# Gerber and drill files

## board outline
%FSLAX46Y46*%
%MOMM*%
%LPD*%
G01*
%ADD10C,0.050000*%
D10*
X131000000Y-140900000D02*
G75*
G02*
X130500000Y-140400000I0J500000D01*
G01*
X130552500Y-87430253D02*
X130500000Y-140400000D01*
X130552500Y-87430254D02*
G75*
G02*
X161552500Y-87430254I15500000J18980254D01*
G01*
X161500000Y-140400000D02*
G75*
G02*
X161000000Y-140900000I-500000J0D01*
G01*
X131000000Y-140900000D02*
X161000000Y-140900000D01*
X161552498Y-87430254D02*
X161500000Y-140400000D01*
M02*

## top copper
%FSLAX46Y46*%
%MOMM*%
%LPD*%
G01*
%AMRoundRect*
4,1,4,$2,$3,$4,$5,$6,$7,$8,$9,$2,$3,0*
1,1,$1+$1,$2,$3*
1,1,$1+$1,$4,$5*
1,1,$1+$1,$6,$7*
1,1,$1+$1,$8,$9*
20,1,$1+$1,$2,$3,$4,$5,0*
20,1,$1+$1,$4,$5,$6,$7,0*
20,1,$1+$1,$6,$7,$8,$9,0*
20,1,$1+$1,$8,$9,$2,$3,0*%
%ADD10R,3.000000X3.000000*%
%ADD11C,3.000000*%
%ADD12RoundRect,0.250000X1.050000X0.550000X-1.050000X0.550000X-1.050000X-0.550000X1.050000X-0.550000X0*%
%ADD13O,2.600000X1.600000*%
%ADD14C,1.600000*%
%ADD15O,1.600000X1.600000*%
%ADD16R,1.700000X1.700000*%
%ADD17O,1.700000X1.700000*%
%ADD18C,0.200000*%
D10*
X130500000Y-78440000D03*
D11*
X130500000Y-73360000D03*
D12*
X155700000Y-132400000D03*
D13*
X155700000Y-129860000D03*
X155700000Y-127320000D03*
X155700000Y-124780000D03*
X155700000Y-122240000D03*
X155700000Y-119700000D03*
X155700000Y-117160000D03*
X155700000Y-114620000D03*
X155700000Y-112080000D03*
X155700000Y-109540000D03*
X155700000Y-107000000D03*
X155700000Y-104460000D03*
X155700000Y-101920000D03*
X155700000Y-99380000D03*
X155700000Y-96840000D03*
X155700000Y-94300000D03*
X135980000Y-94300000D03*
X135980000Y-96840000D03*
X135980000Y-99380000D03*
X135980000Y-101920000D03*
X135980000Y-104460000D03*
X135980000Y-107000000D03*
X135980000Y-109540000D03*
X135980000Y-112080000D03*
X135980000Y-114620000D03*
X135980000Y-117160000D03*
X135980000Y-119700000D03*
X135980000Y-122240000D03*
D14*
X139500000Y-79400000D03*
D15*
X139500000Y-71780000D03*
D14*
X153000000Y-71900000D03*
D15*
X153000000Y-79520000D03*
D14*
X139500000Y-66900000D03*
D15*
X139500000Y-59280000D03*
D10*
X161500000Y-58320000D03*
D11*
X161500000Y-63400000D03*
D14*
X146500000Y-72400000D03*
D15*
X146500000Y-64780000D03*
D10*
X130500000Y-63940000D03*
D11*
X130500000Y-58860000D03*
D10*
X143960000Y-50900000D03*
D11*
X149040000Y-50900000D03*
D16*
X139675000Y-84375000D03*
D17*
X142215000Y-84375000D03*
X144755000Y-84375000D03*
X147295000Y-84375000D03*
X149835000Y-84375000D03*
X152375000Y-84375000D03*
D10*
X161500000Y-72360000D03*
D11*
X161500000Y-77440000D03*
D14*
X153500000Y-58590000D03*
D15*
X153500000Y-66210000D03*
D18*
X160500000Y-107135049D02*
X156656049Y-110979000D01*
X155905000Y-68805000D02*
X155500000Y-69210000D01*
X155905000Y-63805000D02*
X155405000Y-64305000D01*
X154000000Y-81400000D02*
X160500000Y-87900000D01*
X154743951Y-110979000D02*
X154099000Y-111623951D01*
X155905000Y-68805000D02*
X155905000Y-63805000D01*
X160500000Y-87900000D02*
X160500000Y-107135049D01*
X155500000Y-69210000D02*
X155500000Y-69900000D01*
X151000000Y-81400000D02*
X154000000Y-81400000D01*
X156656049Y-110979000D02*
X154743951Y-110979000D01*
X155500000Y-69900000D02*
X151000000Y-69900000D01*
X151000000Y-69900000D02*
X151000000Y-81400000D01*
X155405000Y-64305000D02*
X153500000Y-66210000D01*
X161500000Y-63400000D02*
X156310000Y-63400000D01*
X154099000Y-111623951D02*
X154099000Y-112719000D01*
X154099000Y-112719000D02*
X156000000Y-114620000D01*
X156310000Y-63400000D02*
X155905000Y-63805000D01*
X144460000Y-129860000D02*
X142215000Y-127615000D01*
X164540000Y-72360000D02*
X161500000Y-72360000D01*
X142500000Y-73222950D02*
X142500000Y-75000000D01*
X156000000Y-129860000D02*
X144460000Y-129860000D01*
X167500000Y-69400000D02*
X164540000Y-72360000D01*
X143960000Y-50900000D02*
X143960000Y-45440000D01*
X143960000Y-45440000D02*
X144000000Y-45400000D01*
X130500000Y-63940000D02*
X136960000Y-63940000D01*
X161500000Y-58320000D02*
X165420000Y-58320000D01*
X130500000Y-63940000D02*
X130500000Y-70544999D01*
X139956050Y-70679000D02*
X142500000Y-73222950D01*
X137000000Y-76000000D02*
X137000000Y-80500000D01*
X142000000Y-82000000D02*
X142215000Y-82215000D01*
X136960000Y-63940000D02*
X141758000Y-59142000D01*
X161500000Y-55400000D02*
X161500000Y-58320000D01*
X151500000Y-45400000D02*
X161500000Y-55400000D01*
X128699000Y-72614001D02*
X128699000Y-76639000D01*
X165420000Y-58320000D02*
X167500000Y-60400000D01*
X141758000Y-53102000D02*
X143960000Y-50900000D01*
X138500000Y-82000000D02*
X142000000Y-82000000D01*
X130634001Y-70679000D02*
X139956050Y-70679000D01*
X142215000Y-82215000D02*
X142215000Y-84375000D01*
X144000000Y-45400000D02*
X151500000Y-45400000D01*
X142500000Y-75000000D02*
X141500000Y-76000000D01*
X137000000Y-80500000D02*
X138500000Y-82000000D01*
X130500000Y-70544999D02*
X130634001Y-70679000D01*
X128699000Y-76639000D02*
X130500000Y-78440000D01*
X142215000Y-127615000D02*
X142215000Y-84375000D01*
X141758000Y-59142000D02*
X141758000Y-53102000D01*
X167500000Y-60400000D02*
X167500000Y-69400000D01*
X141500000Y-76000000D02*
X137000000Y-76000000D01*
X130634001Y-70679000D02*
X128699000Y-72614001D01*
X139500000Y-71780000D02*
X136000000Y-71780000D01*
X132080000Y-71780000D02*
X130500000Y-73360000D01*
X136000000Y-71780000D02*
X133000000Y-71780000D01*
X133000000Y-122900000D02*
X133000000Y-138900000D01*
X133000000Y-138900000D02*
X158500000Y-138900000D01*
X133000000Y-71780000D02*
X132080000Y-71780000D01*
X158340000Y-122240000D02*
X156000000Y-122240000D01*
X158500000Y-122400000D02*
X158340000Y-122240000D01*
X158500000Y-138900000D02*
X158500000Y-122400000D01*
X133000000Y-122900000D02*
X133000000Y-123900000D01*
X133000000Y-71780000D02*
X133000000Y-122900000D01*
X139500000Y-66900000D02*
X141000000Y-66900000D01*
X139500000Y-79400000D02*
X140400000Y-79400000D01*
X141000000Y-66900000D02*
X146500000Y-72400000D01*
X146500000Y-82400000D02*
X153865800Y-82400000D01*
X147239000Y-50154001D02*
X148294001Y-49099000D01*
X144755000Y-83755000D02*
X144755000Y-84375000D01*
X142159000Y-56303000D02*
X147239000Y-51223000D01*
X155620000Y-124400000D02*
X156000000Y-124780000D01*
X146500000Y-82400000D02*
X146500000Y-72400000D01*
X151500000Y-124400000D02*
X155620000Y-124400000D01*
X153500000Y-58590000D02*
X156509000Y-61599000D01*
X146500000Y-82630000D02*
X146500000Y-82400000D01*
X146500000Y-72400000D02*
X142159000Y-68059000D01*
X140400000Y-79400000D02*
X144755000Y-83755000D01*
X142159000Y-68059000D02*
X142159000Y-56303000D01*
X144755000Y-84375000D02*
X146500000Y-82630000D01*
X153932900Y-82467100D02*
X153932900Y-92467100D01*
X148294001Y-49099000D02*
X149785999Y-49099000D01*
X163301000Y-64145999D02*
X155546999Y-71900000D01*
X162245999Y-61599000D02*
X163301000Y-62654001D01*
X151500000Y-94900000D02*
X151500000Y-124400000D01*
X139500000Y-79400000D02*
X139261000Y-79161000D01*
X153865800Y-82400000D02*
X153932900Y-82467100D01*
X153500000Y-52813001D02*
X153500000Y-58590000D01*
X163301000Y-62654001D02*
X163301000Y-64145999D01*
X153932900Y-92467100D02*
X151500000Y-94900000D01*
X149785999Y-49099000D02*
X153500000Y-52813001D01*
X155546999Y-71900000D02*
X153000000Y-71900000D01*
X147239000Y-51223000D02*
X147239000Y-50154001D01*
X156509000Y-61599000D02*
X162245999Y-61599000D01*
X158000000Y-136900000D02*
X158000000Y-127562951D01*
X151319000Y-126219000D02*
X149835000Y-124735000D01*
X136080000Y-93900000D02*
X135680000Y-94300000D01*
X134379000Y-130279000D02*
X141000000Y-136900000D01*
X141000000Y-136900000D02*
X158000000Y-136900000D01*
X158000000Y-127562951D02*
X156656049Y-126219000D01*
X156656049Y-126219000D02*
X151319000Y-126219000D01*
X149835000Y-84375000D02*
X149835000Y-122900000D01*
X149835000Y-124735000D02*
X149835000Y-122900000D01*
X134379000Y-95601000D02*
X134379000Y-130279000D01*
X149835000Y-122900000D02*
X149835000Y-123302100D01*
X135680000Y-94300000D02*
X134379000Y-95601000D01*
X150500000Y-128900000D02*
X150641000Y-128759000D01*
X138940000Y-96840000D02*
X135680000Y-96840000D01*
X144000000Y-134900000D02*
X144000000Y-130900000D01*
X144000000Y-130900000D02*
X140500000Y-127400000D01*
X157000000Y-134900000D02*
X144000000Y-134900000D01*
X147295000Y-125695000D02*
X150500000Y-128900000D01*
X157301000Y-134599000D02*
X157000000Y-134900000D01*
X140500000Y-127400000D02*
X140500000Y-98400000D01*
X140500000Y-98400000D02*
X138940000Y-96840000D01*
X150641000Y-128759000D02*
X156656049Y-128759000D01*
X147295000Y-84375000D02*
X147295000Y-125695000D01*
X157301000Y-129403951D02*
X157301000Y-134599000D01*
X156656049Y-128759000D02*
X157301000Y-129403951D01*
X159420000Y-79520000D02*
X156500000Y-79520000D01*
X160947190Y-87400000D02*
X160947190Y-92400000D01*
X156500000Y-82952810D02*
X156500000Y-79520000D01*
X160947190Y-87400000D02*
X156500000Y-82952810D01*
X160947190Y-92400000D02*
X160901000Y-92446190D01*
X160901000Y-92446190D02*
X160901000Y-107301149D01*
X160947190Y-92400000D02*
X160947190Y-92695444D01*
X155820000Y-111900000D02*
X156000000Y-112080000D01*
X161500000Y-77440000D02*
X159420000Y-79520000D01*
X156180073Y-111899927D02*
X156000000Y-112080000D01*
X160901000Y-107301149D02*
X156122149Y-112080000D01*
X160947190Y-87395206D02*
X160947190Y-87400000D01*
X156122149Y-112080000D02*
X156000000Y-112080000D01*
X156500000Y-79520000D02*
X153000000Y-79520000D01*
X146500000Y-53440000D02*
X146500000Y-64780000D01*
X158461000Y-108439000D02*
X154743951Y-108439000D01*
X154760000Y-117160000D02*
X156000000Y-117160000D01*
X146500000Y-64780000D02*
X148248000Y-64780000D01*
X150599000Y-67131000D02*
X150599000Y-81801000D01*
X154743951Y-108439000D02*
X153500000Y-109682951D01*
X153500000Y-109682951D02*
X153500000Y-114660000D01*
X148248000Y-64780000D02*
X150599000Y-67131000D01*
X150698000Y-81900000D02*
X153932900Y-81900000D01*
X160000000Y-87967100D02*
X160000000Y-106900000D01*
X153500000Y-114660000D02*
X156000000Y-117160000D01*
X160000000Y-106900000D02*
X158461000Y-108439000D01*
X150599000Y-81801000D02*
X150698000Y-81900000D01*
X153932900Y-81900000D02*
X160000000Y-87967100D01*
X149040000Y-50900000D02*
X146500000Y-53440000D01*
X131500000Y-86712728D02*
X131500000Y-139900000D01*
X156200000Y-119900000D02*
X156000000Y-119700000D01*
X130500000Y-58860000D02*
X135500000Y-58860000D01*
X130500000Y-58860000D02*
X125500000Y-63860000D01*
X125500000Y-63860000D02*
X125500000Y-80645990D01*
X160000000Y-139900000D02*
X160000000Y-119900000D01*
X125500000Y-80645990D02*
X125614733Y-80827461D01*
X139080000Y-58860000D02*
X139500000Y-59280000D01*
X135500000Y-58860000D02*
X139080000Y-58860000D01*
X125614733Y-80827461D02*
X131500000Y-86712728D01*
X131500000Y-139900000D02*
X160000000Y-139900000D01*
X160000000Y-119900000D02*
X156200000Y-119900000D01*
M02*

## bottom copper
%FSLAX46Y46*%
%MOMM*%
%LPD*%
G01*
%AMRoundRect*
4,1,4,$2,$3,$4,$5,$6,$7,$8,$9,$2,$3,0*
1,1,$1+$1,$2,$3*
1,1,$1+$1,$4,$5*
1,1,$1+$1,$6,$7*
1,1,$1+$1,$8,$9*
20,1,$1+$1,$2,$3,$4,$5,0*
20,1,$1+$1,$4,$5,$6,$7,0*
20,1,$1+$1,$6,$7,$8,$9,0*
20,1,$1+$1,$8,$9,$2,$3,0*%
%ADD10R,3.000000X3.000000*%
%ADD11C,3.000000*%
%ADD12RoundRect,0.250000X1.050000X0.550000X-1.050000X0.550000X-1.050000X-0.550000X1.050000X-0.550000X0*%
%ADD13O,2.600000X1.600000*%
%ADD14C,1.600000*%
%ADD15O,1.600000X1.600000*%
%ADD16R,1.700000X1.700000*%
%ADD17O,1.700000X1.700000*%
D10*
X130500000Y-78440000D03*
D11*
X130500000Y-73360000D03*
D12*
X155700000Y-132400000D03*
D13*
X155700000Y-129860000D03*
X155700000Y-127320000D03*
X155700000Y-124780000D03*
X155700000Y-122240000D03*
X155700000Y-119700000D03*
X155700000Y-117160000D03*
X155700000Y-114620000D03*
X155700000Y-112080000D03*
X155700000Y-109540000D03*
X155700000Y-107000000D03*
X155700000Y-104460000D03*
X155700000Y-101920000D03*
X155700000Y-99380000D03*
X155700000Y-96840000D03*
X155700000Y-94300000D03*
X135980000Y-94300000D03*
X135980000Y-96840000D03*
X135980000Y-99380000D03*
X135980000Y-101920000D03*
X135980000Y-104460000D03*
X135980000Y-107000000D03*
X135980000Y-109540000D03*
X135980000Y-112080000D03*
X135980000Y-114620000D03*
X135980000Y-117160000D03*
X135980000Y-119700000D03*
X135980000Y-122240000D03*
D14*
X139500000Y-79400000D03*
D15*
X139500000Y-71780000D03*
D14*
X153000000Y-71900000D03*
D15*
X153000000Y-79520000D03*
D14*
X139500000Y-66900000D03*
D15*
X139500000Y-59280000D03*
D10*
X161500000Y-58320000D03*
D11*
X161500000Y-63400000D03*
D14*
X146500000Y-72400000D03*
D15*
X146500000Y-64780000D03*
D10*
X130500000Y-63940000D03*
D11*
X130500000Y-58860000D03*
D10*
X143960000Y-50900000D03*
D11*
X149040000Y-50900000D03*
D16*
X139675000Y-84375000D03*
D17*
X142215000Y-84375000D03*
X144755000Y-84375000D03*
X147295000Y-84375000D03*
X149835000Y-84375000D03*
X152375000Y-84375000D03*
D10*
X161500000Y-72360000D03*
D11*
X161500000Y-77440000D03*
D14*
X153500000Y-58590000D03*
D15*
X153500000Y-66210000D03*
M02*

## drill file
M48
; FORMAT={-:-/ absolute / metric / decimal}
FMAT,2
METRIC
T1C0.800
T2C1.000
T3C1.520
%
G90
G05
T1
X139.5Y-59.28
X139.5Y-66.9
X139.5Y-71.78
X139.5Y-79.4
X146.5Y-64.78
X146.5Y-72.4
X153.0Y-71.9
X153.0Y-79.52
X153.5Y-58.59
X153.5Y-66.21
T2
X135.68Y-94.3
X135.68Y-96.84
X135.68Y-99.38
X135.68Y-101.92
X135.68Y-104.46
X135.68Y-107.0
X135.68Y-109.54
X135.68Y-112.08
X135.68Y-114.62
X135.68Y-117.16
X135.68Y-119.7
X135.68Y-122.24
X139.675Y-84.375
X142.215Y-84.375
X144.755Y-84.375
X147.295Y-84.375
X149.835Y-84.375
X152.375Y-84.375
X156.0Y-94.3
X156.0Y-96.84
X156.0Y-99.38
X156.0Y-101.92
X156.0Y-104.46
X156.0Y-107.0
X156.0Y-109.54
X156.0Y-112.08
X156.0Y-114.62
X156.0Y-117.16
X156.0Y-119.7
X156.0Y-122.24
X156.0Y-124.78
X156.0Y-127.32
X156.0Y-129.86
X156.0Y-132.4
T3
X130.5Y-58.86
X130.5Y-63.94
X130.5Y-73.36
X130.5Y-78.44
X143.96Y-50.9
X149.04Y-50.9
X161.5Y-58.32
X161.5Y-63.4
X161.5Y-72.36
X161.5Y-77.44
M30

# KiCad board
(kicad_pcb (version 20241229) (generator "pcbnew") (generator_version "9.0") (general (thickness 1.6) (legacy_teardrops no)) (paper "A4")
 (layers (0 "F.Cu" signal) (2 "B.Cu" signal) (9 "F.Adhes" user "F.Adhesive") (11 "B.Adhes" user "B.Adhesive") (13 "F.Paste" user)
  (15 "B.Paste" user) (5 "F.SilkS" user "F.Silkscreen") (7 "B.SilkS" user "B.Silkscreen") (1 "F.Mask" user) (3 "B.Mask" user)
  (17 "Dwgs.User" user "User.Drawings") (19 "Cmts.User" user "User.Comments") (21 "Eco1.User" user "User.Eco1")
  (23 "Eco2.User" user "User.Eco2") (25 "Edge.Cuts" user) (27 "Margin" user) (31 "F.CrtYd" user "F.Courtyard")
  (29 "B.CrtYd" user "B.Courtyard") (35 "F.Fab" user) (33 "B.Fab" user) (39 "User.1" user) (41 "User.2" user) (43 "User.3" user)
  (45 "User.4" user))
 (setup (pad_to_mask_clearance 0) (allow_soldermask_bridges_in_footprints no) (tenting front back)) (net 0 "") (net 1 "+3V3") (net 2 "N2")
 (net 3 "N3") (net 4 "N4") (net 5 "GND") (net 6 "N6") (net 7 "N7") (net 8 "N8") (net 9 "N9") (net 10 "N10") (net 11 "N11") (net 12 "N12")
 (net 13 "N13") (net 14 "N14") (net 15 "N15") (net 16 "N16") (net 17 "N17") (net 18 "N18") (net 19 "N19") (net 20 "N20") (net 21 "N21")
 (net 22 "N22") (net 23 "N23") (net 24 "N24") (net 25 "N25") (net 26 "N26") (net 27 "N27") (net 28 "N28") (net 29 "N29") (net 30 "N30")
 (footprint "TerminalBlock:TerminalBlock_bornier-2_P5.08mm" (layer "F.Cu") (at 130.5 78.44 90)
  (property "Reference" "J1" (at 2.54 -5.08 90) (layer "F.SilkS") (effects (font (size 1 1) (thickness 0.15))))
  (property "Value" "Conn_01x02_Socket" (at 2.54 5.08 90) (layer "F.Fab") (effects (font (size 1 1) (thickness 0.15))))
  (pad "1" thru_hole rect (at 0 0 90) (size 3 3) (drill 1.52) (layers "*.Cu" "*.Mask") (remove_unused_layers no) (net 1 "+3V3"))
  (pad "2" thru_hole circle (at 5.08 0 90) (size 3 3) (drill 1.52) (layers "*.Cu" "*.Mask") (remove_unused_layers no) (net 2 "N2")))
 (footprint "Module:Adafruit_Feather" (layer "F.Cu") (at 156 132.4 180)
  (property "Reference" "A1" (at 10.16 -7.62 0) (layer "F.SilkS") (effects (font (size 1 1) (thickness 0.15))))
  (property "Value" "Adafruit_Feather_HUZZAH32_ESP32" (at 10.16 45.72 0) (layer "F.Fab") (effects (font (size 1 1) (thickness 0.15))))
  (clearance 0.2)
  (pad "1" thru_hole roundrect (at 0 0 180) (size 2.6 1.6) (drill 1 (offset 0.3 0)) (layers "*.Cu" "*.Mask") (remove_unused_layers no)
   (roundrect_rratio 0.15625) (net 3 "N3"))
  (pad "2" thru_hole oval (at 0 2.54 180) (size 2.6 1.6) (drill 1 (offset 0.3 0)) (layers "*.Cu" "*.Mask") (remove_unused_layers no)
   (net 1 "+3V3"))
  (pad "3" thru_hole oval (at 0 5.08 180) (size 2.6 1.6) (drill 1 (offset 0.3 0)) (layers "*.Cu" "*.Mask") (remove_unused_layers no)
   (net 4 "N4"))
  (pad "4" thru_hole oval (at 0 7.62 180) (size 2.6 1.6) (drill 1 (offset 0.3 0)) (layers "*.Cu" "*.Mask") (remove_unused_layers no)
   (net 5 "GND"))
  (pad "5" thru_hole oval (at 0 10.16 180) (size 2.6 1.6) (drill 1 (offset 0.3 0)) (layers "*.Cu" "*.Mask") (remove_unused_layers no)
   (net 2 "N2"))
  (pad "6" thru_hole oval (at 0 12.7 180) (size 2.6 1.6) (drill 1 (offset 0.3 0)) (layers "*.Cu" "*.Mask") (remove_unused_layers no)
   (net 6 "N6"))
  (pad "7" thru_hole oval (at 0 15.24 180) (size 2.6 1.6) (drill 1 (offset 0.3 0)) (layers "*.Cu" "*.Mask") (remove_unused_layers no)
   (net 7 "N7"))
  (pad "8" thru_hole oval (at 0 17.78 180) (size 2.6 1.6) (drill 1 (offset 0.3 0)) (layers "*.Cu" "*.Mask") (remove_unused_layers no)
   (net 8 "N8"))
  (pad "9" thru_hole oval (at 0 20.32 180) (size 2.6 1.6) (drill 1 (offset 0.3 0)) (layers "*.Cu" "*.Mask") (remove_unused_layers no)
   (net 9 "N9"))
  (pad "10" thru_hole oval (at 0 22.86 180) (size 2.6 1.6) (drill 1 (offset 0.3 0)) (layers "*.Cu" "*.Mask") (remove_unused_layers no)
   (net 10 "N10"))
  (pad "11" thru_hole oval (at 0 25.4 180) (size 2.6 1.6) (drill 1 (offset 0.3 0)) (layers "*.Cu" "*.Mask") (remove_unused_layers no)
   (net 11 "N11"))
  (pad "12" thru_hole oval (at 0 27.94 180) (size 2.6 1.6) (drill 1 (offset 0.3 0)) (layers "*.Cu" "*.Mask") (remove_unused_layers no)
   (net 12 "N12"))
  (pad "13" thru_hole oval (at 0 30.48 180) (size 2.6 1.6) (drill 1 (offset 0.3 0)) (layers "*.Cu" "*.Mask") (remove_unused_layers no)
   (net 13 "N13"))
  (pad "14" thru_hole oval (at 0 33.02 180) (size 2.6 1.6) (drill 1 (offset 0.3 0)) (layers "*.Cu" "*.Mask") (remove_unused_layers no)
   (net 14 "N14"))
  (pad "15" thru_hole oval (at 0 35.56 180) (size 2.6 1.6) (drill 1 (offset 0.3 0)) (layers "*.Cu" "*.Mask") (remove_unused_layers no)
   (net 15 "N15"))
  (pad "16" thru_hole oval (at 0 38.1 180) (size 2.6 1.6) (drill 1 (offset 0.3 0)) (layers "*.Cu" "*.Mask") (remove_unused_layers no)
   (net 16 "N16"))
  (pad "17" thru_hole oval (at 20.32 38.1) (size 2.6 1.6) (drill 1 (offset 0.3 0)) (layers "*.Cu" "*.Mask") (remove_unused_layers no)
   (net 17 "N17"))
  (pad "18" thru_hole oval (at 20.32 35.56) (size 2.6 1.6) (drill 1 (offset 0.3 0)) (layers "*.Cu" "*.Mask") (remove_unused_layers no)
   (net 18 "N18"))
  (pad "19" thru_hole oval (at 20.32 33.02) (size 2.6 1.6) (drill 1 (offset 0.3 0)) (layers "*.Cu" "*.Mask") (remove_unused_layers no)
   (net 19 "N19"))
  (pad "20" thru_hole oval (at 20.32 30.48) (size 2.6 1.6) (drill 1 (offset 0.3 0)) (layers "*.Cu" "*.Mask") (remove_unused_layers no)
   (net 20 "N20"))
  (pad "21" thru_hole oval (at 20.32 27.94) (size 2.6 1.6) (drill 1 (offset 0.3 0)) (layers "*.Cu" "*.Mask") (remove_unused_layers no)
   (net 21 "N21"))
  (pad "22" thru_hole oval (at 20.32 25.4) (size 2.6 1.6) (drill 1 (offset 0.3 0)) (layers "*.Cu" "*.Mask") (remove_unused_layers no)
   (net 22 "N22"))
  (pad "23" thru_hole oval (at 20.32 22.86) (size 2.6 1.6) (drill 1 (offset 0.3 0)) (layers "*.Cu" "*.Mask") (remove_unused_layers no)
   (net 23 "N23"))
  (pad "24" thru_hole oval (at 20.32 20.32) (size 2.6 1.6) (drill 1 (offset 0.3 0)) (layers "*.Cu" "*.Mask") (remove_unused_layers no)
   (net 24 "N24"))
  (pad "25" thru_hole oval (at 20.32 17.78) (size 2.6 1.6) (drill 1 (offset 0.3 0)) (layers "*.Cu" "*.Mask") (remove_unused_layers no)
   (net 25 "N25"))
  (pad "26" thru_hole oval (at 20.32 15.24) (size 2.6 1.6) (drill 1 (offset 0.3 0)) (layers "*.Cu" "*.Mask") (remove_unused_layers no)
   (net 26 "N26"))
  (pad "27" thru_hole oval (at 20.32 12.7) (size 2.6 1.6) (drill 1 (offset 0.3 0)) (layers "*.Cu" "*.Mask") (remove_unused_layers no)
   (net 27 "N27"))
  (pad "28" thru_hole oval (at 20.32 10.16) (size 2.6 1.6) (drill 1 (offset 0.3 0)) (layers "*.Cu" "*.Mask") (remove_unused_layers no)
   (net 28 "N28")))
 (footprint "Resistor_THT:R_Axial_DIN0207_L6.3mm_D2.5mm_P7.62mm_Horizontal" (layer "F.Cu") (at 139.5 79.4 90)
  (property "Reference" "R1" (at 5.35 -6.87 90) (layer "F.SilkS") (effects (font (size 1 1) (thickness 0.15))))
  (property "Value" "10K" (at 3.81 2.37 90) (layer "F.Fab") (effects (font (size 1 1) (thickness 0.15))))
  (pad "1" thru_hole circle (at 0 0 90) (size 1.6 1.6) (drill 0.8) (layers "*.Cu" "*.Mask") (remove_unused_layers no) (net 5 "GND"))
  (pad "2" thru_hole oval (at 7.62 0 90) (size 1.6 1.6) (drill 0.8) (layers "*.Cu" "*.Mask") (remove_unused_layers no) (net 2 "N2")))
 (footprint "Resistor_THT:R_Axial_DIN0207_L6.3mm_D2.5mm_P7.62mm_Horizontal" (layer "F.Cu") (at 153 71.9 -90)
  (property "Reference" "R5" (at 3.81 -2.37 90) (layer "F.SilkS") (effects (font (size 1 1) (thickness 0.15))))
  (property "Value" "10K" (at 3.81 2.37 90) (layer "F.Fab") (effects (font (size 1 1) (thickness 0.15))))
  (pad "1" thru_hole circle (at 0 0 270) (size 1.6 1.6) (drill 0.8) (layers "*.Cu" "*.Mask") (remove_unused_layers no) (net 5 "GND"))
  (pad "2" thru_hole oval (at 7.62 0 270) (size 1.6 1.6) (drill 0.8) (layers "*.Cu" "*.Mask") (remove_unused_layers no) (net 9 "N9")))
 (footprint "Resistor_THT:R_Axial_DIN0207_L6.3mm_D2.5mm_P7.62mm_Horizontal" (layer "F.Cu") (at 139.5 66.9 90)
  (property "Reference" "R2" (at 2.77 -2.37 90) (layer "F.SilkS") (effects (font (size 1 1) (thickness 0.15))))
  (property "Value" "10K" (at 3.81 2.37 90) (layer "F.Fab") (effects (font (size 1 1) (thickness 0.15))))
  (pad "1" thru_hole circle (at 0 0 90) (size 1.6 1.6) (drill 0.8) (layers "*.Cu" "*.Mask") (remove_unused_layers no) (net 5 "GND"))
  (pad "2" thru_hole oval (at 7.62 0 90) (size 1.6 1.6) (drill 0.8) (layers "*.Cu" "*.Mask") (remove_unused_layers no) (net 6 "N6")))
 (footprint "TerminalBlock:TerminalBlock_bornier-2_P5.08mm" (layer "F.Cu") (at 161.5 58.32 -90)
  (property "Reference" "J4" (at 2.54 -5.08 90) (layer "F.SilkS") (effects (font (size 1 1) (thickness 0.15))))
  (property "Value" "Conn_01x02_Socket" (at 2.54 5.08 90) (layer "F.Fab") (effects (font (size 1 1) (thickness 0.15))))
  (pad "1" thru_hole rect (at 0 0 270) (size 3 3) (drill 1.52) (layers "*.Cu" "*.Mask") (remove_unused_layers no) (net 1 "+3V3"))
  (pad "2" thru_hole circle (at 5.08 0 270) (size 3 3) (drill 1.52) (layers "*.Cu" "*.Mask") (remove_unused_layers no) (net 8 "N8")))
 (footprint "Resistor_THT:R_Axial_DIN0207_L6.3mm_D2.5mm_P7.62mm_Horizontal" (layer "F.Cu") (at 146.5 72.4 90)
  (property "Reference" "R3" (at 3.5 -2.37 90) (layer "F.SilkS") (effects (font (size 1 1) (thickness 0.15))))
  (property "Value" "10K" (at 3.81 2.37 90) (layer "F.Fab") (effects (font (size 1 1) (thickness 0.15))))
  (pad "1" thru_hole circle (at 0 0 90) (size 1.6 1.6) (drill 0.8) (layers "*.Cu" "*.Mask") (remove_unused_layers no) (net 5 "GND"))
  (pad "2" thru_hole oval (at 7.62 0 90) (size 1.6 1.6) (drill 0.8) (layers "*.Cu" "*.Mask") (remove_unused_layers no) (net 7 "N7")))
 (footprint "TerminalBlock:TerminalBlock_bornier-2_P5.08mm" (layer "F.Cu") (at 130.5 63.94 90)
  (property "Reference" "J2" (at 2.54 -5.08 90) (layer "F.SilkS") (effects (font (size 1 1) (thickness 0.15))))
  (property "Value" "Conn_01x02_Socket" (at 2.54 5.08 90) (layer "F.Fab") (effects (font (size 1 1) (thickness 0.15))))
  (pad "1" thru_hole rect (at 0 0 90) (size 3 3) (drill 1.52) (layers "*.Cu" "*.Mask") (remove_unused_layers no) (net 1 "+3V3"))
  (pad "2" thru_hole circle (at 5.08 0 90) (size 3 3) (drill 1.52) (layers "*.Cu" "*.Mask") (remove_unused_layers no) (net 6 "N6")))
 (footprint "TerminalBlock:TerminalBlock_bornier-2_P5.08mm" (layer "F.Cu") (at 143.96 50.9)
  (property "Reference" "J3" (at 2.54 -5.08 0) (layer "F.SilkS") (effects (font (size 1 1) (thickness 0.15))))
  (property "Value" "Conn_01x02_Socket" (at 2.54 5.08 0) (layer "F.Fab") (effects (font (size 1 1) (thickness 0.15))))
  (pad "1" thru_hole rect (at 0 0) (size 3 3) (drill 1.52) (layers "*.Cu" "*.Mask") (remove_unused_layers no) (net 1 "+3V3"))
  (pad "2" thru_hole circle (at 5.08 0) (size 3 3) (drill 1.52) (layers "*.Cu" "*.Mask") (remove_unused_layers no) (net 7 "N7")))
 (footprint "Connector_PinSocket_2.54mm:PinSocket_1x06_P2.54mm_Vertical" (layer "F.Cu") (at 139.675 84.375 90)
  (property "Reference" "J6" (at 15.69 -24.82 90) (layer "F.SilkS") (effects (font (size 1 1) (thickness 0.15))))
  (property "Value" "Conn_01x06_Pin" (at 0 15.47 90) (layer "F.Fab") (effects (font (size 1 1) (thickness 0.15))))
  (pad "1" thru_hole rect (at 0 0 90) (size 1.7 1.7) (drill 1) (layers "*.Cu" "*.Mask") (remove_unused_layers no) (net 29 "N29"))
  (pad "2" thru_hole oval (at 0 2.54 90) (size 1.7 1.7) (drill 1) (layers "*.Cu" "*.Mask") (remove_unused_layers no) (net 1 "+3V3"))
  (pad "3" thru_hole oval (at 0 5.08 90) (size 1.7 1.7) (drill 1) (layers "*.Cu" "*.Mask") (remove_unused_layers no) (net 5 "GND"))
  (pad "4" thru_hole oval (at 0 7.62 90) (size 1.7 1.7) (drill 1) (layers "*.Cu" "*.Mask") (remove_unused_layers no) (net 18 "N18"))
  (pad "5" thru_hole oval (at 0 10.16 90) (size 1.7 1.7) (drill 1) (layers "*.Cu" "*.Mask") (remove_unused_layers no) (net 17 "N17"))
  (pad "6" thru_hole oval (at 0 12.7 90) (size 1.7 1.7) (drill 1) (layers "*.Cu" "*.Mask") (remove_unused_layers no) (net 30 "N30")))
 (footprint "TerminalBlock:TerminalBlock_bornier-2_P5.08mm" (layer "F.Cu") (at 161.5 72.36 -90)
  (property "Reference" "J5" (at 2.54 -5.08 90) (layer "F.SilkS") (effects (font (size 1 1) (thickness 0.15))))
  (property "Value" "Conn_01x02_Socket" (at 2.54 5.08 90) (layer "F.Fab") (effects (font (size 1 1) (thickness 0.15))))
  (pad "1" thru_hole rect (at 0 0 270) (size 3 3) (drill 1.52) (layers "*.Cu" "*.Mask") (remove_unused_layers no) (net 1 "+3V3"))
  (pad "2" thru_hole circle (at 5.08 0 270) (size 3 3) (drill 1.52) (layers "*.Cu" "*.Mask") (remove_unused_layers no) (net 9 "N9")))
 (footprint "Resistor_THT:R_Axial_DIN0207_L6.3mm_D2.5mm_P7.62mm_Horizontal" (layer "F.Cu") (at 153.5 58.59 -90)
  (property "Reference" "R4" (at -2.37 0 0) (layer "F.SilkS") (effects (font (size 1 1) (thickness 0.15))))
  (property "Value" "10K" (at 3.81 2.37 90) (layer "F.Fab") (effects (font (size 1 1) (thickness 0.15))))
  (pad "1" thru_hole circle (at 0 0 270) (size 1.6 1.6) (drill 0.8) (layers "*.Cu" "*.Mask") (remove_unused_layers no) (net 5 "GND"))
  (pad "2" thru_hole oval (at 7.62 0 270) (size 1.6 1.6) (drill 0.8) (layers "*.Cu" "*.Mask") (remove_unused_layers no) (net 8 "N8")))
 (gr_arc (start 131 140.9) (mid 130.646447 140.753553) (end 130.5 140.4) (stroke (width 0.05) (type default)) (layer "Edge.Cuts"))
 (gr_line (start 130.5525 87.430253) (end 130.5 140.4) (stroke (width 0.05) (type default)) (layer "Edge.Cuts"))
 (gr_arc (start 130.5525 87.430254) (mid 146.0525 43.944898) (end 161.5525 87.430254) (stroke (width 0.05) (type default))
  (layer "Edge.Cuts"))
 (gr_arc (start 161.5 140.4) (mid 161.353553 140.753553) (end 161 140.9) (stroke (width 0.05) (type default)) (layer "Edge.Cuts"))
 (gr_line (start 131 140.9) (end 161 140.9) (stroke (width 0.05) (type default)) (layer "Edge.Cuts"))
 (gr_line (start 161.552498 87.430254) (end 161.5 140.4) (stroke (width 0.05) (type default)) (layer "Edge.Cuts"))
 (segment (start 160.5 107.135049) (end 156.656049 110.979) (width 0.2) (layer "F.Cu") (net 8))
 (segment (start 155.905 68.805) (end 155.5 69.21) (width 0.2) (layer "F.Cu") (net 8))
 (segment (start 155.905 63.805) (end 155.405 64.305) (width 0.2) (layer "F.Cu") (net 8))
 (segment (start 154 81.4) (end 160.5 87.9) (width 0.2) (layer "F.Cu") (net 8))
 (segment (start 154.743951 110.979) (end 154.099 111.623951) (width 0.2) (layer "F.Cu") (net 8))
 (segment (start 155.905 68.805) (end 155.905 63.805) (width 0.2) (layer "F.Cu") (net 8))
 (segment (start 160.5 87.9) (end 160.5 107.135049) (width 0.2) (layer "F.Cu") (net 8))
 (segment (start 155.5 69.21) (end 155.5 69.9) (width 0.2) (layer "F.Cu") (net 8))
 (segment (start 151 81.4) (end 154 81.4) (width 0.2) (layer "F.Cu") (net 8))
 (segment (start 156.656049 110.979) (end 154.743951 110.979) (width 0.2) (layer "F.Cu") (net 8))
 (segment (start 155.5 69.9) (end 151 69.9) (width 0.2) (layer "F.Cu") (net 8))
 (segment (start 151 69.9) (end 151 81.4) (width 0.2) (layer "F.Cu") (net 8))
 (segment (start 155.405 64.305) (end 153.5 66.21) (width 0.2) (layer "F.Cu") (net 8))
 (segment (start 161.5 63.4) (end 156.31 63.4) (width 0.2) (layer "F.Cu") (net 8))
 (segment (start 154.099 111.623951) (end 154.099 112.719) (width 0.2) (layer "F.Cu") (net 8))
 (segment (start 154.099 112.719) (end 156 114.62) (width 0.2) (layer "F.Cu") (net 8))
 (segment (start 156.31 63.4) (end 155.905 63.805) (width 0.2) (layer "F.Cu") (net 8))
 (segment (start 144.46 129.86) (end 142.215 127.615) (width 0.2) (layer "F.Cu") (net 1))
 (segment (start 164.54 72.36) (end 161.5 72.36) (width 0.2) (layer "F.Cu") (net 1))
 (segment (start 142.5 73.22295) (end 142.5 75) (width 0.2) (layer "F.Cu") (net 1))
 (segment (start 156 129.86) (end 144.46 129.86) (width 0.2) (layer "F.Cu") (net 1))
 (segment (start 167.5 69.4) (end 164.54 72.36) (width 0.2) (layer "F.Cu") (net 1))
 (segment (start 143.96 50.9) (end 143.96 45.44) (width 0.2) (layer "F.Cu") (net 1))
 (segment (start 143.96 45.44) (end 144 45.4) (width 0.2) (layer "F.Cu") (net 1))
 (segment (start 130.5 63.94) (end 136.96 63.94) (width 0.2) (layer "F.Cu") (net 1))
 (segment (start 161.5 58.32) (end 165.42 58.32) (width 0.2) (layer "F.Cu") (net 1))
 (segment (start 130.5 63.94) (end 130.5 70.544999) (width 0.2) (layer "F.Cu") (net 1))
 (segment (start 139.95605 70.679) (end 142.5 73.22295) (width 0.2) (layer "F.Cu") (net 1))
 (segment (start 137 76) (end 137 80.5) (width 0.2) (layer "F.Cu") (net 1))
 (segment (start 142 82) (end 142.215 82.215) (width 0.2) (layer "F.Cu") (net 1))
 (segment (start 136.96 63.94) (end 141.758 59.142) (width 0.2) (layer "F.Cu") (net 1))
 (segment (start 161.5 55.4) (end 161.5 58.32) (width 0.2) (layer "F.Cu") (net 1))
 (segment (start 151.5 45.4) (end 161.5 55.4) (width 0.2) (layer "F.Cu") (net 1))
 (segment (start 128.699 72.614001) (end 128.699 76.639) (width 0.2) (layer "F.Cu") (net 1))
 (segment (start 165.42 58.32) (end 167.5 60.4) (width 0.2) (layer "F.Cu") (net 1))
 (segment (start 141.758 53.102) (end 143.96 50.9) (width 0.2) (layer "F.Cu") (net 1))
 (segment (start 138.5 82) (end 142 82) (width 0.2) (layer "F.Cu") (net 1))
 (segment (start 130.634001 70.679) (end 139.95605 70.679) (width 0.2) (layer "F.Cu") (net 1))
 (segment (start 142.215 82.215) (end 142.215 84.375) (width 0.2) (layer "F.Cu") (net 1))
 (segment (start 144 45.4) (end 151.5 45.4) (width 0.2) (layer "F.Cu") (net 1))
 (segment (start 142.5 75) (end 141.5 76) (width 0.2) (layer "F.Cu") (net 1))
 (segment (start 137 80.5) (end 138.5 82) (width 0.2) (layer "F.Cu") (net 1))
 (segment (start 130.5 70.544999) (end 130.634001 70.679) (width 0.2) (layer "F.Cu") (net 1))
 (segment (start 128.699 76.639) (end 130.5 78.44) (width 0.2) (layer "F.Cu") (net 1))
 (segment (start 142.215 127.615) (end 142.215 84.375) (width 0.2) (layer "F.Cu") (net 1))
 (segment (start 141.758 59.142) (end 141.758 53.102) (width 0.2) (layer "F.Cu") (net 1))
 (segment (start 167.5 60.4) (end 167.5 69.4) (width 0.2) (layer "F.Cu") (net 1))
 (segment (start 141.5 76) (end 137 76) (width 0.2) (layer "F.Cu") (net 1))
 (segment (start 130.634001 70.679) (end 128.699 72.614001) (width 0.2) (layer "F.Cu") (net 1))
 (segment (start 139.5 71.78) (end 136 71.78) (width 0.2) (layer "F.Cu") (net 2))
 (segment (start 132.08 71.78) (end 130.5 73.36) (width 0.2) (layer "F.Cu") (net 2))
 (segment (start 136 71.78) (end 133 71.78) (width 0.2) (layer "F.Cu") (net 2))
 (segment (start 133 122.9) (end 133 138.9) (width 0.2) (layer "F.Cu") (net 2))
 (segment (start 133 138.9) (end 158.5 138.9) (width 0.2) (layer "F.Cu") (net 2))
 (segment (start 133 71.78) (end 132.08 71.78) (width 0.2) (layer "F.Cu") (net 2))
 (segment (start 158.34 122.24) (end 156 122.24) (width 0.2) (layer "F.Cu") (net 2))
 (segment (start 158.5 122.4) (end 158.34 122.24) (width 0.2) (layer "F.Cu") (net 2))
 (segment (start 158.5 138.9) (end 158.5 122.4) (width 0.2) (layer "F.Cu") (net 2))
 (segment (start 133 122.9) (end 133 123.9) (width 0.2) (layer "F.Cu") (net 2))
 (segment (start 133 71.78) (end 133 122.9) (width 0.2) (layer "F.Cu") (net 2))
 (segment (start 139.5 66.9) (end 141 66.9) (width 0.2) (layer "F.Cu") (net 5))
 (segment (start 139.5 79.4) (end 140.4 79.4) (width 0.2) (layer "F.Cu") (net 5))
 (segment (start 141 66.9) (end 146.5 72.4) (width 0.2) (layer "F.Cu") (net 5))
 (segment (start 146.5 82.4) (end 153.8658 82.4) (width 0.2) (layer "F.Cu") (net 5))
 (segment (start 147.239 50.154001) (end 148.294001 49.099) (width 0.2) (layer "F.Cu") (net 5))
 (segment (start 144.755 83.755) (end 144.755 84.375) (width 0.2) (layer "F.Cu") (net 5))
 (segment (start 142.159 56.303) (end 147.239 51.223) (width 0.2) (layer "F.Cu") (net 5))
 (segment (start 155.62 124.4) (end 156 124.78) (width 0.2) (layer "F.Cu") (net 5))
 (segment (start 146.5 82.4) (end 146.5 72.4) (width 0.2) (layer "F.Cu") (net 5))
 (segment (start 151.5 124.4) (end 155.62 124.4) (width 0.2) (layer "F.Cu") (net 5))
 (segment (start 153.5 58.59) (end 156.509 61.599) (width 0.2) (layer "F.Cu") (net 5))
 (segment (start 146.5 82.63) (end 146.5 82.4) (width 0.2) (layer "F.Cu") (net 5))
 (segment (start 146.5 72.4) (end 142.159 68.059) (width 0.2) (layer "F.Cu") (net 5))
 (segment (start 140.4 79.4) (end 144.755 83.755) (width 0.2) (layer "F.Cu") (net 5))
 (segment (start 142.159 68.059) (end 142.159 56.303) (width 0.2) (layer "F.Cu") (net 5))
 (segment (start 144.755 84.375) (end 146.5 82.63) (width 0.2) (layer "F.Cu") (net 5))
 (segment (start 153.9329 82.4671) (end 153.9329 92.4671) (width 0.2) (layer "F.Cu") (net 5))
 (segment (start 148.294001 49.099) (end 149.785999 49.099) (width 0.2) (layer "F.Cu") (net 5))
 (segment (start 163.301 64.145999) (end 155.546999 71.9) (width 0.2) (layer "F.Cu") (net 5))
 (segment (start 162.245999 61.599) (end 163.301 62.654001) (width 0.2) (layer "F.Cu") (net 5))
 (segment (start 151.5 94.9) (end 151.5 124.4) (width 0.2) (layer "F.Cu") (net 5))
 (segment (start 139.5 79.4) (end 139.261 79.161) (width 0.2) (layer "F.Cu") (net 5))
 (segment (start 153.8658 82.4) (end 153.9329 82.4671) (width 0.2) (layer "F.Cu") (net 5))
 (segment (start 153.5 52.813001) (end 153.5 58.59) (width 0.2) (layer "F.Cu") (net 5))
 (segment (start 163.301 62.654001) (end 163.301 64.145999) (width 0.2) (layer "F.Cu") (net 5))
 (segment (start 153.9329 92.4671) (end 151.5 94.9) (width 0.2) (layer "F.Cu") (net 5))
 (segment (start 149.785999 49.099) (end 153.5 52.813001) (width 0.2) (layer "F.Cu") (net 5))
 (segment (start 155.546999 71.9) (end 153 71.9) (width 0.2) (layer "F.Cu") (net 5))
 (segment (start 147.239 51.223) (end 147.239 50.154001) (width 0.2) (layer "F.Cu") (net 5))
 (segment (start 156.509 61.599) (end 162.245999 61.599) (width 0.2) (layer "F.Cu") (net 5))
 (segment (start 158 136.9) (end 158 127.562951) (width 0.2) (layer "F.Cu") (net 17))
 (segment (start 151.319 126.219) (end 149.835 124.735) (width 0.2) (layer "F.Cu") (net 17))
 (segment (start 136.08 93.9) (end 135.68 94.3) (width 0.2) (layer "F.Cu") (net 17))
 (segment (start 134.379 130.279) (end 141 136.9) (width 0.2) (layer "F.Cu") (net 17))
 (segment (start 141 136.9) (end 158 136.9) (width 0.2) (layer "F.Cu") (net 17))
 (segment (start 158 127.562951) (end 156.656049 126.219) (width 0.2) (layer "F.Cu") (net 17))
 (segment (start 156.656049 126.219) (end 151.319 126.219) (width 0.2) (layer "F.Cu") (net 17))
 (segment (start 149.835 84.375) (end 149.835 122.9) (width 0.2) (layer "F.Cu") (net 17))
 (segment (start 149.835 124.735) (end 149.835 122.9) (width 0.2) (layer "F.Cu") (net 17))
 (segment (start 134.379 95.601) (end 134.379 130.279) (width 0.2) (layer "F.Cu") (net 17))
 (segment (start 149.835 122.9) (end 149.835 123.3021) (width 0.2) (layer "F.Cu") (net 17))
 (segment (start 135.68 94.3) (end 134.379 95.601) (width 0.2) (layer "F.Cu") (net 17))
 (segment (start 150.5 128.9) (end 150.641 128.759) (width 0.2) (layer "F.Cu") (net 18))
 (segment (start 138.94 96.84) (end 135.68 96.84) (width 0.2) (layer "F.Cu") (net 18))
 (segment (start 144 134.9) (end 144 130.9) (width 0.2) (layer "F.Cu") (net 18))
 (segment (start 144 130.9) (end 140.5 127.4) (width 0.2) (layer "F.Cu") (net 18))
 (segment (start 157 134.9) (end 144 134.9) (width 0.2) (layer "F.Cu") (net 18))
 (segment (start 147.295 125.695) (end 150.5 128.9) (width 0.2) (layer "F.Cu") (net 18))
 (segment (start 157.301 134.599) (end 157 134.9) (width 0.2) (layer "F.Cu") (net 18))
 (segment (start 140.5 127.4) (end 140.5 98.4) (width 0.2) (layer "F.Cu") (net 18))
 (segment (start 140.5 98.4) (end 138.94 96.84) (width 0.2) (layer "F.Cu") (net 18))
 (segment (start 150.641 128.759) (end 156.656049 128.759) (width 0.2) (layer "F.Cu") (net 18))
 (segment (start 147.295 84.375) (end 147.295 125.695) (width 0.2) (layer "F.Cu") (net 18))
 (segment (start 157.301 129.403951) (end 157.301 134.599) (width 0.2) (layer "F.Cu") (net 18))
 (segment (start 156.656049 128.759) (end 157.301 129.403951) (width 0.2) (layer "F.Cu") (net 18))
 (segment (start 159.42 79.52) (end 156.5 79.52) (width 0.2) (layer "F.Cu") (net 9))
 (segment (start 160.94719 87.4) (end 160.94719 92.4) (width 0.2) (layer "F.Cu") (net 9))
 (segment (start 156.5 82.95281) (end 156.5 79.52) (width 0.2) (layer "F.Cu") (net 9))
 (segment (start 160.94719 87.4) (end 156.5 82.95281) (width 0.2) (layer "F.Cu") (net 9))
 (segment (start 160.94719 92.4) (end 160.901 92.44619) (width 0.2) (layer "F.Cu") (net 9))
 (segment (start 160.901 92.44619) (end 160.901 107.301149) (width 0.2) (layer "F.Cu") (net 9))
 (segment (start 160.94719 92.4) (end 160.94719 92.695444) (width 0.2) (layer "F.Cu") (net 9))
 (segment (start 155.82 111.9) (end 156 112.08) (width 0.2) (layer "F.Cu") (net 9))
 (segment (start 161.5 77.44) (end 159.42 79.52) (width 0.2) (layer "F.Cu") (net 9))
 (segment (start 156.180073 111.899927) (end 156 112.08) (width 0.2) (layer "F.Cu") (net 9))
 (segment (start 160.901 107.301149) (end 156.122149 112.08) (width 0.2) (layer "F.Cu") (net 9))
 (segment (start 160.94719 87.395206) (end 160.94719 87.4) (width 0.2) (layer "F.Cu") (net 9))
 (segment (start 156.122149 112.08) (end 156 112.08) (width 0.2) (layer "F.Cu") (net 9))
 (segment (start 156.5 79.52) (end 153 79.52) (width 0.2) (layer "F.Cu") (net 9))
 (segment (start 146.5 53.44) (end 146.5 64.78) (width 0.2) (layer "F.Cu") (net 7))
 (segment (start 158.461 108.439) (end 154.743951 108.439) (width 0.2) (layer "F.Cu") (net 7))
 (segment (start 154.76 117.16) (end 156 117.16) (width 0.2) (layer "F.Cu") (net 7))
 (segment (start 146.5 64.78) (end 148.248 64.78) (width 0.2) (layer "F.Cu") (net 7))
 (segment (start 150.599 67.131) (end 150.599 81.801) (width 0.2) (layer "F.Cu") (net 7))
 (segment (start 154.743951 108.439) (end 153.5 109.682951) (width 0.2) (layer "F.Cu") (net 7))
 (segment (start 153.5 109.682951) (end 153.5 114.66) (width 0.2) (layer "F.Cu") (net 7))
 (segment (start 148.248 64.78) (end 150.599 67.131) (width 0.2) (layer "F.Cu") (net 7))
 (segment (start 150.698 81.9) (end 153.9329 81.9) (width 0.2) (layer "F.Cu") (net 7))
 (segment (start 160 87.9671) (end 160 106.9) (width 0.2) (layer "F.Cu") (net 7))
 (segment (start 153.5 114.66) (end 156 117.16) (width 0.2) (layer "F.Cu") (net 7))
 (segment (start 160 106.9) (end 158.461 108.439) (width 0.2) (layer "F.Cu") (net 7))
 (segment (start 150.599 81.801) (end 150.698 81.9) (width 0.2) (layer "F.Cu") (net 7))
 (segment (start 153.9329 81.9) (end 160 87.9671) (width 0.2) (layer "F.Cu") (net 7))
 (segment (start 149.04 50.9) (end 146.5 53.44) (width 0.2) (layer "F.Cu") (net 7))
 (segment (start 131.5 86.712728) (end 131.5 139.9) (width 0.2) (layer "F.Cu") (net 6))
 (segment (start 156.2 119.9) (end 156 119.7) (width 0.2) (layer "F.Cu") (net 6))
 (segment (start 130.5 58.86) (end 135.5 58.86) (width 0.2) (layer "F.Cu") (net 6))
 (segment (start 130.5 58.86) (end 125.5 63.86) (width 0.2) (layer "F.Cu") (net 6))
 (segment (start 125.5 63.86) (end 125.5 80.64599) (width 0.2) (layer "F.Cu") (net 6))
 (segment (start 160 139.9) (end 160 119.9) (width 0.2) (layer "F.Cu") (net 6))
 (segment (start 125.5 80.64599) (end 125.614733 80.827461) (width 0.2) (layer "F.Cu") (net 6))
 (segment (start 139.08 58.86) (end 139.5 59.28) (width 0.2) (layer "F.Cu") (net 6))
 (segment (start 135.5 58.86) (end 139.08 58.86) (width 0.2) (layer "F.Cu") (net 6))
 (segment (start 125.614733 80.827461) (end 131.5 86.712728) (width 0.2) (layer "F.Cu") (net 6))
 (segment (start 131.5 139.9) (end 160 139.9) (width 0.2) (layer "F.Cu") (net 6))
 (segment (start 160 119.9) (end 156.2 119.9) (width 0.2) (layer "F.Cu") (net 6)))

